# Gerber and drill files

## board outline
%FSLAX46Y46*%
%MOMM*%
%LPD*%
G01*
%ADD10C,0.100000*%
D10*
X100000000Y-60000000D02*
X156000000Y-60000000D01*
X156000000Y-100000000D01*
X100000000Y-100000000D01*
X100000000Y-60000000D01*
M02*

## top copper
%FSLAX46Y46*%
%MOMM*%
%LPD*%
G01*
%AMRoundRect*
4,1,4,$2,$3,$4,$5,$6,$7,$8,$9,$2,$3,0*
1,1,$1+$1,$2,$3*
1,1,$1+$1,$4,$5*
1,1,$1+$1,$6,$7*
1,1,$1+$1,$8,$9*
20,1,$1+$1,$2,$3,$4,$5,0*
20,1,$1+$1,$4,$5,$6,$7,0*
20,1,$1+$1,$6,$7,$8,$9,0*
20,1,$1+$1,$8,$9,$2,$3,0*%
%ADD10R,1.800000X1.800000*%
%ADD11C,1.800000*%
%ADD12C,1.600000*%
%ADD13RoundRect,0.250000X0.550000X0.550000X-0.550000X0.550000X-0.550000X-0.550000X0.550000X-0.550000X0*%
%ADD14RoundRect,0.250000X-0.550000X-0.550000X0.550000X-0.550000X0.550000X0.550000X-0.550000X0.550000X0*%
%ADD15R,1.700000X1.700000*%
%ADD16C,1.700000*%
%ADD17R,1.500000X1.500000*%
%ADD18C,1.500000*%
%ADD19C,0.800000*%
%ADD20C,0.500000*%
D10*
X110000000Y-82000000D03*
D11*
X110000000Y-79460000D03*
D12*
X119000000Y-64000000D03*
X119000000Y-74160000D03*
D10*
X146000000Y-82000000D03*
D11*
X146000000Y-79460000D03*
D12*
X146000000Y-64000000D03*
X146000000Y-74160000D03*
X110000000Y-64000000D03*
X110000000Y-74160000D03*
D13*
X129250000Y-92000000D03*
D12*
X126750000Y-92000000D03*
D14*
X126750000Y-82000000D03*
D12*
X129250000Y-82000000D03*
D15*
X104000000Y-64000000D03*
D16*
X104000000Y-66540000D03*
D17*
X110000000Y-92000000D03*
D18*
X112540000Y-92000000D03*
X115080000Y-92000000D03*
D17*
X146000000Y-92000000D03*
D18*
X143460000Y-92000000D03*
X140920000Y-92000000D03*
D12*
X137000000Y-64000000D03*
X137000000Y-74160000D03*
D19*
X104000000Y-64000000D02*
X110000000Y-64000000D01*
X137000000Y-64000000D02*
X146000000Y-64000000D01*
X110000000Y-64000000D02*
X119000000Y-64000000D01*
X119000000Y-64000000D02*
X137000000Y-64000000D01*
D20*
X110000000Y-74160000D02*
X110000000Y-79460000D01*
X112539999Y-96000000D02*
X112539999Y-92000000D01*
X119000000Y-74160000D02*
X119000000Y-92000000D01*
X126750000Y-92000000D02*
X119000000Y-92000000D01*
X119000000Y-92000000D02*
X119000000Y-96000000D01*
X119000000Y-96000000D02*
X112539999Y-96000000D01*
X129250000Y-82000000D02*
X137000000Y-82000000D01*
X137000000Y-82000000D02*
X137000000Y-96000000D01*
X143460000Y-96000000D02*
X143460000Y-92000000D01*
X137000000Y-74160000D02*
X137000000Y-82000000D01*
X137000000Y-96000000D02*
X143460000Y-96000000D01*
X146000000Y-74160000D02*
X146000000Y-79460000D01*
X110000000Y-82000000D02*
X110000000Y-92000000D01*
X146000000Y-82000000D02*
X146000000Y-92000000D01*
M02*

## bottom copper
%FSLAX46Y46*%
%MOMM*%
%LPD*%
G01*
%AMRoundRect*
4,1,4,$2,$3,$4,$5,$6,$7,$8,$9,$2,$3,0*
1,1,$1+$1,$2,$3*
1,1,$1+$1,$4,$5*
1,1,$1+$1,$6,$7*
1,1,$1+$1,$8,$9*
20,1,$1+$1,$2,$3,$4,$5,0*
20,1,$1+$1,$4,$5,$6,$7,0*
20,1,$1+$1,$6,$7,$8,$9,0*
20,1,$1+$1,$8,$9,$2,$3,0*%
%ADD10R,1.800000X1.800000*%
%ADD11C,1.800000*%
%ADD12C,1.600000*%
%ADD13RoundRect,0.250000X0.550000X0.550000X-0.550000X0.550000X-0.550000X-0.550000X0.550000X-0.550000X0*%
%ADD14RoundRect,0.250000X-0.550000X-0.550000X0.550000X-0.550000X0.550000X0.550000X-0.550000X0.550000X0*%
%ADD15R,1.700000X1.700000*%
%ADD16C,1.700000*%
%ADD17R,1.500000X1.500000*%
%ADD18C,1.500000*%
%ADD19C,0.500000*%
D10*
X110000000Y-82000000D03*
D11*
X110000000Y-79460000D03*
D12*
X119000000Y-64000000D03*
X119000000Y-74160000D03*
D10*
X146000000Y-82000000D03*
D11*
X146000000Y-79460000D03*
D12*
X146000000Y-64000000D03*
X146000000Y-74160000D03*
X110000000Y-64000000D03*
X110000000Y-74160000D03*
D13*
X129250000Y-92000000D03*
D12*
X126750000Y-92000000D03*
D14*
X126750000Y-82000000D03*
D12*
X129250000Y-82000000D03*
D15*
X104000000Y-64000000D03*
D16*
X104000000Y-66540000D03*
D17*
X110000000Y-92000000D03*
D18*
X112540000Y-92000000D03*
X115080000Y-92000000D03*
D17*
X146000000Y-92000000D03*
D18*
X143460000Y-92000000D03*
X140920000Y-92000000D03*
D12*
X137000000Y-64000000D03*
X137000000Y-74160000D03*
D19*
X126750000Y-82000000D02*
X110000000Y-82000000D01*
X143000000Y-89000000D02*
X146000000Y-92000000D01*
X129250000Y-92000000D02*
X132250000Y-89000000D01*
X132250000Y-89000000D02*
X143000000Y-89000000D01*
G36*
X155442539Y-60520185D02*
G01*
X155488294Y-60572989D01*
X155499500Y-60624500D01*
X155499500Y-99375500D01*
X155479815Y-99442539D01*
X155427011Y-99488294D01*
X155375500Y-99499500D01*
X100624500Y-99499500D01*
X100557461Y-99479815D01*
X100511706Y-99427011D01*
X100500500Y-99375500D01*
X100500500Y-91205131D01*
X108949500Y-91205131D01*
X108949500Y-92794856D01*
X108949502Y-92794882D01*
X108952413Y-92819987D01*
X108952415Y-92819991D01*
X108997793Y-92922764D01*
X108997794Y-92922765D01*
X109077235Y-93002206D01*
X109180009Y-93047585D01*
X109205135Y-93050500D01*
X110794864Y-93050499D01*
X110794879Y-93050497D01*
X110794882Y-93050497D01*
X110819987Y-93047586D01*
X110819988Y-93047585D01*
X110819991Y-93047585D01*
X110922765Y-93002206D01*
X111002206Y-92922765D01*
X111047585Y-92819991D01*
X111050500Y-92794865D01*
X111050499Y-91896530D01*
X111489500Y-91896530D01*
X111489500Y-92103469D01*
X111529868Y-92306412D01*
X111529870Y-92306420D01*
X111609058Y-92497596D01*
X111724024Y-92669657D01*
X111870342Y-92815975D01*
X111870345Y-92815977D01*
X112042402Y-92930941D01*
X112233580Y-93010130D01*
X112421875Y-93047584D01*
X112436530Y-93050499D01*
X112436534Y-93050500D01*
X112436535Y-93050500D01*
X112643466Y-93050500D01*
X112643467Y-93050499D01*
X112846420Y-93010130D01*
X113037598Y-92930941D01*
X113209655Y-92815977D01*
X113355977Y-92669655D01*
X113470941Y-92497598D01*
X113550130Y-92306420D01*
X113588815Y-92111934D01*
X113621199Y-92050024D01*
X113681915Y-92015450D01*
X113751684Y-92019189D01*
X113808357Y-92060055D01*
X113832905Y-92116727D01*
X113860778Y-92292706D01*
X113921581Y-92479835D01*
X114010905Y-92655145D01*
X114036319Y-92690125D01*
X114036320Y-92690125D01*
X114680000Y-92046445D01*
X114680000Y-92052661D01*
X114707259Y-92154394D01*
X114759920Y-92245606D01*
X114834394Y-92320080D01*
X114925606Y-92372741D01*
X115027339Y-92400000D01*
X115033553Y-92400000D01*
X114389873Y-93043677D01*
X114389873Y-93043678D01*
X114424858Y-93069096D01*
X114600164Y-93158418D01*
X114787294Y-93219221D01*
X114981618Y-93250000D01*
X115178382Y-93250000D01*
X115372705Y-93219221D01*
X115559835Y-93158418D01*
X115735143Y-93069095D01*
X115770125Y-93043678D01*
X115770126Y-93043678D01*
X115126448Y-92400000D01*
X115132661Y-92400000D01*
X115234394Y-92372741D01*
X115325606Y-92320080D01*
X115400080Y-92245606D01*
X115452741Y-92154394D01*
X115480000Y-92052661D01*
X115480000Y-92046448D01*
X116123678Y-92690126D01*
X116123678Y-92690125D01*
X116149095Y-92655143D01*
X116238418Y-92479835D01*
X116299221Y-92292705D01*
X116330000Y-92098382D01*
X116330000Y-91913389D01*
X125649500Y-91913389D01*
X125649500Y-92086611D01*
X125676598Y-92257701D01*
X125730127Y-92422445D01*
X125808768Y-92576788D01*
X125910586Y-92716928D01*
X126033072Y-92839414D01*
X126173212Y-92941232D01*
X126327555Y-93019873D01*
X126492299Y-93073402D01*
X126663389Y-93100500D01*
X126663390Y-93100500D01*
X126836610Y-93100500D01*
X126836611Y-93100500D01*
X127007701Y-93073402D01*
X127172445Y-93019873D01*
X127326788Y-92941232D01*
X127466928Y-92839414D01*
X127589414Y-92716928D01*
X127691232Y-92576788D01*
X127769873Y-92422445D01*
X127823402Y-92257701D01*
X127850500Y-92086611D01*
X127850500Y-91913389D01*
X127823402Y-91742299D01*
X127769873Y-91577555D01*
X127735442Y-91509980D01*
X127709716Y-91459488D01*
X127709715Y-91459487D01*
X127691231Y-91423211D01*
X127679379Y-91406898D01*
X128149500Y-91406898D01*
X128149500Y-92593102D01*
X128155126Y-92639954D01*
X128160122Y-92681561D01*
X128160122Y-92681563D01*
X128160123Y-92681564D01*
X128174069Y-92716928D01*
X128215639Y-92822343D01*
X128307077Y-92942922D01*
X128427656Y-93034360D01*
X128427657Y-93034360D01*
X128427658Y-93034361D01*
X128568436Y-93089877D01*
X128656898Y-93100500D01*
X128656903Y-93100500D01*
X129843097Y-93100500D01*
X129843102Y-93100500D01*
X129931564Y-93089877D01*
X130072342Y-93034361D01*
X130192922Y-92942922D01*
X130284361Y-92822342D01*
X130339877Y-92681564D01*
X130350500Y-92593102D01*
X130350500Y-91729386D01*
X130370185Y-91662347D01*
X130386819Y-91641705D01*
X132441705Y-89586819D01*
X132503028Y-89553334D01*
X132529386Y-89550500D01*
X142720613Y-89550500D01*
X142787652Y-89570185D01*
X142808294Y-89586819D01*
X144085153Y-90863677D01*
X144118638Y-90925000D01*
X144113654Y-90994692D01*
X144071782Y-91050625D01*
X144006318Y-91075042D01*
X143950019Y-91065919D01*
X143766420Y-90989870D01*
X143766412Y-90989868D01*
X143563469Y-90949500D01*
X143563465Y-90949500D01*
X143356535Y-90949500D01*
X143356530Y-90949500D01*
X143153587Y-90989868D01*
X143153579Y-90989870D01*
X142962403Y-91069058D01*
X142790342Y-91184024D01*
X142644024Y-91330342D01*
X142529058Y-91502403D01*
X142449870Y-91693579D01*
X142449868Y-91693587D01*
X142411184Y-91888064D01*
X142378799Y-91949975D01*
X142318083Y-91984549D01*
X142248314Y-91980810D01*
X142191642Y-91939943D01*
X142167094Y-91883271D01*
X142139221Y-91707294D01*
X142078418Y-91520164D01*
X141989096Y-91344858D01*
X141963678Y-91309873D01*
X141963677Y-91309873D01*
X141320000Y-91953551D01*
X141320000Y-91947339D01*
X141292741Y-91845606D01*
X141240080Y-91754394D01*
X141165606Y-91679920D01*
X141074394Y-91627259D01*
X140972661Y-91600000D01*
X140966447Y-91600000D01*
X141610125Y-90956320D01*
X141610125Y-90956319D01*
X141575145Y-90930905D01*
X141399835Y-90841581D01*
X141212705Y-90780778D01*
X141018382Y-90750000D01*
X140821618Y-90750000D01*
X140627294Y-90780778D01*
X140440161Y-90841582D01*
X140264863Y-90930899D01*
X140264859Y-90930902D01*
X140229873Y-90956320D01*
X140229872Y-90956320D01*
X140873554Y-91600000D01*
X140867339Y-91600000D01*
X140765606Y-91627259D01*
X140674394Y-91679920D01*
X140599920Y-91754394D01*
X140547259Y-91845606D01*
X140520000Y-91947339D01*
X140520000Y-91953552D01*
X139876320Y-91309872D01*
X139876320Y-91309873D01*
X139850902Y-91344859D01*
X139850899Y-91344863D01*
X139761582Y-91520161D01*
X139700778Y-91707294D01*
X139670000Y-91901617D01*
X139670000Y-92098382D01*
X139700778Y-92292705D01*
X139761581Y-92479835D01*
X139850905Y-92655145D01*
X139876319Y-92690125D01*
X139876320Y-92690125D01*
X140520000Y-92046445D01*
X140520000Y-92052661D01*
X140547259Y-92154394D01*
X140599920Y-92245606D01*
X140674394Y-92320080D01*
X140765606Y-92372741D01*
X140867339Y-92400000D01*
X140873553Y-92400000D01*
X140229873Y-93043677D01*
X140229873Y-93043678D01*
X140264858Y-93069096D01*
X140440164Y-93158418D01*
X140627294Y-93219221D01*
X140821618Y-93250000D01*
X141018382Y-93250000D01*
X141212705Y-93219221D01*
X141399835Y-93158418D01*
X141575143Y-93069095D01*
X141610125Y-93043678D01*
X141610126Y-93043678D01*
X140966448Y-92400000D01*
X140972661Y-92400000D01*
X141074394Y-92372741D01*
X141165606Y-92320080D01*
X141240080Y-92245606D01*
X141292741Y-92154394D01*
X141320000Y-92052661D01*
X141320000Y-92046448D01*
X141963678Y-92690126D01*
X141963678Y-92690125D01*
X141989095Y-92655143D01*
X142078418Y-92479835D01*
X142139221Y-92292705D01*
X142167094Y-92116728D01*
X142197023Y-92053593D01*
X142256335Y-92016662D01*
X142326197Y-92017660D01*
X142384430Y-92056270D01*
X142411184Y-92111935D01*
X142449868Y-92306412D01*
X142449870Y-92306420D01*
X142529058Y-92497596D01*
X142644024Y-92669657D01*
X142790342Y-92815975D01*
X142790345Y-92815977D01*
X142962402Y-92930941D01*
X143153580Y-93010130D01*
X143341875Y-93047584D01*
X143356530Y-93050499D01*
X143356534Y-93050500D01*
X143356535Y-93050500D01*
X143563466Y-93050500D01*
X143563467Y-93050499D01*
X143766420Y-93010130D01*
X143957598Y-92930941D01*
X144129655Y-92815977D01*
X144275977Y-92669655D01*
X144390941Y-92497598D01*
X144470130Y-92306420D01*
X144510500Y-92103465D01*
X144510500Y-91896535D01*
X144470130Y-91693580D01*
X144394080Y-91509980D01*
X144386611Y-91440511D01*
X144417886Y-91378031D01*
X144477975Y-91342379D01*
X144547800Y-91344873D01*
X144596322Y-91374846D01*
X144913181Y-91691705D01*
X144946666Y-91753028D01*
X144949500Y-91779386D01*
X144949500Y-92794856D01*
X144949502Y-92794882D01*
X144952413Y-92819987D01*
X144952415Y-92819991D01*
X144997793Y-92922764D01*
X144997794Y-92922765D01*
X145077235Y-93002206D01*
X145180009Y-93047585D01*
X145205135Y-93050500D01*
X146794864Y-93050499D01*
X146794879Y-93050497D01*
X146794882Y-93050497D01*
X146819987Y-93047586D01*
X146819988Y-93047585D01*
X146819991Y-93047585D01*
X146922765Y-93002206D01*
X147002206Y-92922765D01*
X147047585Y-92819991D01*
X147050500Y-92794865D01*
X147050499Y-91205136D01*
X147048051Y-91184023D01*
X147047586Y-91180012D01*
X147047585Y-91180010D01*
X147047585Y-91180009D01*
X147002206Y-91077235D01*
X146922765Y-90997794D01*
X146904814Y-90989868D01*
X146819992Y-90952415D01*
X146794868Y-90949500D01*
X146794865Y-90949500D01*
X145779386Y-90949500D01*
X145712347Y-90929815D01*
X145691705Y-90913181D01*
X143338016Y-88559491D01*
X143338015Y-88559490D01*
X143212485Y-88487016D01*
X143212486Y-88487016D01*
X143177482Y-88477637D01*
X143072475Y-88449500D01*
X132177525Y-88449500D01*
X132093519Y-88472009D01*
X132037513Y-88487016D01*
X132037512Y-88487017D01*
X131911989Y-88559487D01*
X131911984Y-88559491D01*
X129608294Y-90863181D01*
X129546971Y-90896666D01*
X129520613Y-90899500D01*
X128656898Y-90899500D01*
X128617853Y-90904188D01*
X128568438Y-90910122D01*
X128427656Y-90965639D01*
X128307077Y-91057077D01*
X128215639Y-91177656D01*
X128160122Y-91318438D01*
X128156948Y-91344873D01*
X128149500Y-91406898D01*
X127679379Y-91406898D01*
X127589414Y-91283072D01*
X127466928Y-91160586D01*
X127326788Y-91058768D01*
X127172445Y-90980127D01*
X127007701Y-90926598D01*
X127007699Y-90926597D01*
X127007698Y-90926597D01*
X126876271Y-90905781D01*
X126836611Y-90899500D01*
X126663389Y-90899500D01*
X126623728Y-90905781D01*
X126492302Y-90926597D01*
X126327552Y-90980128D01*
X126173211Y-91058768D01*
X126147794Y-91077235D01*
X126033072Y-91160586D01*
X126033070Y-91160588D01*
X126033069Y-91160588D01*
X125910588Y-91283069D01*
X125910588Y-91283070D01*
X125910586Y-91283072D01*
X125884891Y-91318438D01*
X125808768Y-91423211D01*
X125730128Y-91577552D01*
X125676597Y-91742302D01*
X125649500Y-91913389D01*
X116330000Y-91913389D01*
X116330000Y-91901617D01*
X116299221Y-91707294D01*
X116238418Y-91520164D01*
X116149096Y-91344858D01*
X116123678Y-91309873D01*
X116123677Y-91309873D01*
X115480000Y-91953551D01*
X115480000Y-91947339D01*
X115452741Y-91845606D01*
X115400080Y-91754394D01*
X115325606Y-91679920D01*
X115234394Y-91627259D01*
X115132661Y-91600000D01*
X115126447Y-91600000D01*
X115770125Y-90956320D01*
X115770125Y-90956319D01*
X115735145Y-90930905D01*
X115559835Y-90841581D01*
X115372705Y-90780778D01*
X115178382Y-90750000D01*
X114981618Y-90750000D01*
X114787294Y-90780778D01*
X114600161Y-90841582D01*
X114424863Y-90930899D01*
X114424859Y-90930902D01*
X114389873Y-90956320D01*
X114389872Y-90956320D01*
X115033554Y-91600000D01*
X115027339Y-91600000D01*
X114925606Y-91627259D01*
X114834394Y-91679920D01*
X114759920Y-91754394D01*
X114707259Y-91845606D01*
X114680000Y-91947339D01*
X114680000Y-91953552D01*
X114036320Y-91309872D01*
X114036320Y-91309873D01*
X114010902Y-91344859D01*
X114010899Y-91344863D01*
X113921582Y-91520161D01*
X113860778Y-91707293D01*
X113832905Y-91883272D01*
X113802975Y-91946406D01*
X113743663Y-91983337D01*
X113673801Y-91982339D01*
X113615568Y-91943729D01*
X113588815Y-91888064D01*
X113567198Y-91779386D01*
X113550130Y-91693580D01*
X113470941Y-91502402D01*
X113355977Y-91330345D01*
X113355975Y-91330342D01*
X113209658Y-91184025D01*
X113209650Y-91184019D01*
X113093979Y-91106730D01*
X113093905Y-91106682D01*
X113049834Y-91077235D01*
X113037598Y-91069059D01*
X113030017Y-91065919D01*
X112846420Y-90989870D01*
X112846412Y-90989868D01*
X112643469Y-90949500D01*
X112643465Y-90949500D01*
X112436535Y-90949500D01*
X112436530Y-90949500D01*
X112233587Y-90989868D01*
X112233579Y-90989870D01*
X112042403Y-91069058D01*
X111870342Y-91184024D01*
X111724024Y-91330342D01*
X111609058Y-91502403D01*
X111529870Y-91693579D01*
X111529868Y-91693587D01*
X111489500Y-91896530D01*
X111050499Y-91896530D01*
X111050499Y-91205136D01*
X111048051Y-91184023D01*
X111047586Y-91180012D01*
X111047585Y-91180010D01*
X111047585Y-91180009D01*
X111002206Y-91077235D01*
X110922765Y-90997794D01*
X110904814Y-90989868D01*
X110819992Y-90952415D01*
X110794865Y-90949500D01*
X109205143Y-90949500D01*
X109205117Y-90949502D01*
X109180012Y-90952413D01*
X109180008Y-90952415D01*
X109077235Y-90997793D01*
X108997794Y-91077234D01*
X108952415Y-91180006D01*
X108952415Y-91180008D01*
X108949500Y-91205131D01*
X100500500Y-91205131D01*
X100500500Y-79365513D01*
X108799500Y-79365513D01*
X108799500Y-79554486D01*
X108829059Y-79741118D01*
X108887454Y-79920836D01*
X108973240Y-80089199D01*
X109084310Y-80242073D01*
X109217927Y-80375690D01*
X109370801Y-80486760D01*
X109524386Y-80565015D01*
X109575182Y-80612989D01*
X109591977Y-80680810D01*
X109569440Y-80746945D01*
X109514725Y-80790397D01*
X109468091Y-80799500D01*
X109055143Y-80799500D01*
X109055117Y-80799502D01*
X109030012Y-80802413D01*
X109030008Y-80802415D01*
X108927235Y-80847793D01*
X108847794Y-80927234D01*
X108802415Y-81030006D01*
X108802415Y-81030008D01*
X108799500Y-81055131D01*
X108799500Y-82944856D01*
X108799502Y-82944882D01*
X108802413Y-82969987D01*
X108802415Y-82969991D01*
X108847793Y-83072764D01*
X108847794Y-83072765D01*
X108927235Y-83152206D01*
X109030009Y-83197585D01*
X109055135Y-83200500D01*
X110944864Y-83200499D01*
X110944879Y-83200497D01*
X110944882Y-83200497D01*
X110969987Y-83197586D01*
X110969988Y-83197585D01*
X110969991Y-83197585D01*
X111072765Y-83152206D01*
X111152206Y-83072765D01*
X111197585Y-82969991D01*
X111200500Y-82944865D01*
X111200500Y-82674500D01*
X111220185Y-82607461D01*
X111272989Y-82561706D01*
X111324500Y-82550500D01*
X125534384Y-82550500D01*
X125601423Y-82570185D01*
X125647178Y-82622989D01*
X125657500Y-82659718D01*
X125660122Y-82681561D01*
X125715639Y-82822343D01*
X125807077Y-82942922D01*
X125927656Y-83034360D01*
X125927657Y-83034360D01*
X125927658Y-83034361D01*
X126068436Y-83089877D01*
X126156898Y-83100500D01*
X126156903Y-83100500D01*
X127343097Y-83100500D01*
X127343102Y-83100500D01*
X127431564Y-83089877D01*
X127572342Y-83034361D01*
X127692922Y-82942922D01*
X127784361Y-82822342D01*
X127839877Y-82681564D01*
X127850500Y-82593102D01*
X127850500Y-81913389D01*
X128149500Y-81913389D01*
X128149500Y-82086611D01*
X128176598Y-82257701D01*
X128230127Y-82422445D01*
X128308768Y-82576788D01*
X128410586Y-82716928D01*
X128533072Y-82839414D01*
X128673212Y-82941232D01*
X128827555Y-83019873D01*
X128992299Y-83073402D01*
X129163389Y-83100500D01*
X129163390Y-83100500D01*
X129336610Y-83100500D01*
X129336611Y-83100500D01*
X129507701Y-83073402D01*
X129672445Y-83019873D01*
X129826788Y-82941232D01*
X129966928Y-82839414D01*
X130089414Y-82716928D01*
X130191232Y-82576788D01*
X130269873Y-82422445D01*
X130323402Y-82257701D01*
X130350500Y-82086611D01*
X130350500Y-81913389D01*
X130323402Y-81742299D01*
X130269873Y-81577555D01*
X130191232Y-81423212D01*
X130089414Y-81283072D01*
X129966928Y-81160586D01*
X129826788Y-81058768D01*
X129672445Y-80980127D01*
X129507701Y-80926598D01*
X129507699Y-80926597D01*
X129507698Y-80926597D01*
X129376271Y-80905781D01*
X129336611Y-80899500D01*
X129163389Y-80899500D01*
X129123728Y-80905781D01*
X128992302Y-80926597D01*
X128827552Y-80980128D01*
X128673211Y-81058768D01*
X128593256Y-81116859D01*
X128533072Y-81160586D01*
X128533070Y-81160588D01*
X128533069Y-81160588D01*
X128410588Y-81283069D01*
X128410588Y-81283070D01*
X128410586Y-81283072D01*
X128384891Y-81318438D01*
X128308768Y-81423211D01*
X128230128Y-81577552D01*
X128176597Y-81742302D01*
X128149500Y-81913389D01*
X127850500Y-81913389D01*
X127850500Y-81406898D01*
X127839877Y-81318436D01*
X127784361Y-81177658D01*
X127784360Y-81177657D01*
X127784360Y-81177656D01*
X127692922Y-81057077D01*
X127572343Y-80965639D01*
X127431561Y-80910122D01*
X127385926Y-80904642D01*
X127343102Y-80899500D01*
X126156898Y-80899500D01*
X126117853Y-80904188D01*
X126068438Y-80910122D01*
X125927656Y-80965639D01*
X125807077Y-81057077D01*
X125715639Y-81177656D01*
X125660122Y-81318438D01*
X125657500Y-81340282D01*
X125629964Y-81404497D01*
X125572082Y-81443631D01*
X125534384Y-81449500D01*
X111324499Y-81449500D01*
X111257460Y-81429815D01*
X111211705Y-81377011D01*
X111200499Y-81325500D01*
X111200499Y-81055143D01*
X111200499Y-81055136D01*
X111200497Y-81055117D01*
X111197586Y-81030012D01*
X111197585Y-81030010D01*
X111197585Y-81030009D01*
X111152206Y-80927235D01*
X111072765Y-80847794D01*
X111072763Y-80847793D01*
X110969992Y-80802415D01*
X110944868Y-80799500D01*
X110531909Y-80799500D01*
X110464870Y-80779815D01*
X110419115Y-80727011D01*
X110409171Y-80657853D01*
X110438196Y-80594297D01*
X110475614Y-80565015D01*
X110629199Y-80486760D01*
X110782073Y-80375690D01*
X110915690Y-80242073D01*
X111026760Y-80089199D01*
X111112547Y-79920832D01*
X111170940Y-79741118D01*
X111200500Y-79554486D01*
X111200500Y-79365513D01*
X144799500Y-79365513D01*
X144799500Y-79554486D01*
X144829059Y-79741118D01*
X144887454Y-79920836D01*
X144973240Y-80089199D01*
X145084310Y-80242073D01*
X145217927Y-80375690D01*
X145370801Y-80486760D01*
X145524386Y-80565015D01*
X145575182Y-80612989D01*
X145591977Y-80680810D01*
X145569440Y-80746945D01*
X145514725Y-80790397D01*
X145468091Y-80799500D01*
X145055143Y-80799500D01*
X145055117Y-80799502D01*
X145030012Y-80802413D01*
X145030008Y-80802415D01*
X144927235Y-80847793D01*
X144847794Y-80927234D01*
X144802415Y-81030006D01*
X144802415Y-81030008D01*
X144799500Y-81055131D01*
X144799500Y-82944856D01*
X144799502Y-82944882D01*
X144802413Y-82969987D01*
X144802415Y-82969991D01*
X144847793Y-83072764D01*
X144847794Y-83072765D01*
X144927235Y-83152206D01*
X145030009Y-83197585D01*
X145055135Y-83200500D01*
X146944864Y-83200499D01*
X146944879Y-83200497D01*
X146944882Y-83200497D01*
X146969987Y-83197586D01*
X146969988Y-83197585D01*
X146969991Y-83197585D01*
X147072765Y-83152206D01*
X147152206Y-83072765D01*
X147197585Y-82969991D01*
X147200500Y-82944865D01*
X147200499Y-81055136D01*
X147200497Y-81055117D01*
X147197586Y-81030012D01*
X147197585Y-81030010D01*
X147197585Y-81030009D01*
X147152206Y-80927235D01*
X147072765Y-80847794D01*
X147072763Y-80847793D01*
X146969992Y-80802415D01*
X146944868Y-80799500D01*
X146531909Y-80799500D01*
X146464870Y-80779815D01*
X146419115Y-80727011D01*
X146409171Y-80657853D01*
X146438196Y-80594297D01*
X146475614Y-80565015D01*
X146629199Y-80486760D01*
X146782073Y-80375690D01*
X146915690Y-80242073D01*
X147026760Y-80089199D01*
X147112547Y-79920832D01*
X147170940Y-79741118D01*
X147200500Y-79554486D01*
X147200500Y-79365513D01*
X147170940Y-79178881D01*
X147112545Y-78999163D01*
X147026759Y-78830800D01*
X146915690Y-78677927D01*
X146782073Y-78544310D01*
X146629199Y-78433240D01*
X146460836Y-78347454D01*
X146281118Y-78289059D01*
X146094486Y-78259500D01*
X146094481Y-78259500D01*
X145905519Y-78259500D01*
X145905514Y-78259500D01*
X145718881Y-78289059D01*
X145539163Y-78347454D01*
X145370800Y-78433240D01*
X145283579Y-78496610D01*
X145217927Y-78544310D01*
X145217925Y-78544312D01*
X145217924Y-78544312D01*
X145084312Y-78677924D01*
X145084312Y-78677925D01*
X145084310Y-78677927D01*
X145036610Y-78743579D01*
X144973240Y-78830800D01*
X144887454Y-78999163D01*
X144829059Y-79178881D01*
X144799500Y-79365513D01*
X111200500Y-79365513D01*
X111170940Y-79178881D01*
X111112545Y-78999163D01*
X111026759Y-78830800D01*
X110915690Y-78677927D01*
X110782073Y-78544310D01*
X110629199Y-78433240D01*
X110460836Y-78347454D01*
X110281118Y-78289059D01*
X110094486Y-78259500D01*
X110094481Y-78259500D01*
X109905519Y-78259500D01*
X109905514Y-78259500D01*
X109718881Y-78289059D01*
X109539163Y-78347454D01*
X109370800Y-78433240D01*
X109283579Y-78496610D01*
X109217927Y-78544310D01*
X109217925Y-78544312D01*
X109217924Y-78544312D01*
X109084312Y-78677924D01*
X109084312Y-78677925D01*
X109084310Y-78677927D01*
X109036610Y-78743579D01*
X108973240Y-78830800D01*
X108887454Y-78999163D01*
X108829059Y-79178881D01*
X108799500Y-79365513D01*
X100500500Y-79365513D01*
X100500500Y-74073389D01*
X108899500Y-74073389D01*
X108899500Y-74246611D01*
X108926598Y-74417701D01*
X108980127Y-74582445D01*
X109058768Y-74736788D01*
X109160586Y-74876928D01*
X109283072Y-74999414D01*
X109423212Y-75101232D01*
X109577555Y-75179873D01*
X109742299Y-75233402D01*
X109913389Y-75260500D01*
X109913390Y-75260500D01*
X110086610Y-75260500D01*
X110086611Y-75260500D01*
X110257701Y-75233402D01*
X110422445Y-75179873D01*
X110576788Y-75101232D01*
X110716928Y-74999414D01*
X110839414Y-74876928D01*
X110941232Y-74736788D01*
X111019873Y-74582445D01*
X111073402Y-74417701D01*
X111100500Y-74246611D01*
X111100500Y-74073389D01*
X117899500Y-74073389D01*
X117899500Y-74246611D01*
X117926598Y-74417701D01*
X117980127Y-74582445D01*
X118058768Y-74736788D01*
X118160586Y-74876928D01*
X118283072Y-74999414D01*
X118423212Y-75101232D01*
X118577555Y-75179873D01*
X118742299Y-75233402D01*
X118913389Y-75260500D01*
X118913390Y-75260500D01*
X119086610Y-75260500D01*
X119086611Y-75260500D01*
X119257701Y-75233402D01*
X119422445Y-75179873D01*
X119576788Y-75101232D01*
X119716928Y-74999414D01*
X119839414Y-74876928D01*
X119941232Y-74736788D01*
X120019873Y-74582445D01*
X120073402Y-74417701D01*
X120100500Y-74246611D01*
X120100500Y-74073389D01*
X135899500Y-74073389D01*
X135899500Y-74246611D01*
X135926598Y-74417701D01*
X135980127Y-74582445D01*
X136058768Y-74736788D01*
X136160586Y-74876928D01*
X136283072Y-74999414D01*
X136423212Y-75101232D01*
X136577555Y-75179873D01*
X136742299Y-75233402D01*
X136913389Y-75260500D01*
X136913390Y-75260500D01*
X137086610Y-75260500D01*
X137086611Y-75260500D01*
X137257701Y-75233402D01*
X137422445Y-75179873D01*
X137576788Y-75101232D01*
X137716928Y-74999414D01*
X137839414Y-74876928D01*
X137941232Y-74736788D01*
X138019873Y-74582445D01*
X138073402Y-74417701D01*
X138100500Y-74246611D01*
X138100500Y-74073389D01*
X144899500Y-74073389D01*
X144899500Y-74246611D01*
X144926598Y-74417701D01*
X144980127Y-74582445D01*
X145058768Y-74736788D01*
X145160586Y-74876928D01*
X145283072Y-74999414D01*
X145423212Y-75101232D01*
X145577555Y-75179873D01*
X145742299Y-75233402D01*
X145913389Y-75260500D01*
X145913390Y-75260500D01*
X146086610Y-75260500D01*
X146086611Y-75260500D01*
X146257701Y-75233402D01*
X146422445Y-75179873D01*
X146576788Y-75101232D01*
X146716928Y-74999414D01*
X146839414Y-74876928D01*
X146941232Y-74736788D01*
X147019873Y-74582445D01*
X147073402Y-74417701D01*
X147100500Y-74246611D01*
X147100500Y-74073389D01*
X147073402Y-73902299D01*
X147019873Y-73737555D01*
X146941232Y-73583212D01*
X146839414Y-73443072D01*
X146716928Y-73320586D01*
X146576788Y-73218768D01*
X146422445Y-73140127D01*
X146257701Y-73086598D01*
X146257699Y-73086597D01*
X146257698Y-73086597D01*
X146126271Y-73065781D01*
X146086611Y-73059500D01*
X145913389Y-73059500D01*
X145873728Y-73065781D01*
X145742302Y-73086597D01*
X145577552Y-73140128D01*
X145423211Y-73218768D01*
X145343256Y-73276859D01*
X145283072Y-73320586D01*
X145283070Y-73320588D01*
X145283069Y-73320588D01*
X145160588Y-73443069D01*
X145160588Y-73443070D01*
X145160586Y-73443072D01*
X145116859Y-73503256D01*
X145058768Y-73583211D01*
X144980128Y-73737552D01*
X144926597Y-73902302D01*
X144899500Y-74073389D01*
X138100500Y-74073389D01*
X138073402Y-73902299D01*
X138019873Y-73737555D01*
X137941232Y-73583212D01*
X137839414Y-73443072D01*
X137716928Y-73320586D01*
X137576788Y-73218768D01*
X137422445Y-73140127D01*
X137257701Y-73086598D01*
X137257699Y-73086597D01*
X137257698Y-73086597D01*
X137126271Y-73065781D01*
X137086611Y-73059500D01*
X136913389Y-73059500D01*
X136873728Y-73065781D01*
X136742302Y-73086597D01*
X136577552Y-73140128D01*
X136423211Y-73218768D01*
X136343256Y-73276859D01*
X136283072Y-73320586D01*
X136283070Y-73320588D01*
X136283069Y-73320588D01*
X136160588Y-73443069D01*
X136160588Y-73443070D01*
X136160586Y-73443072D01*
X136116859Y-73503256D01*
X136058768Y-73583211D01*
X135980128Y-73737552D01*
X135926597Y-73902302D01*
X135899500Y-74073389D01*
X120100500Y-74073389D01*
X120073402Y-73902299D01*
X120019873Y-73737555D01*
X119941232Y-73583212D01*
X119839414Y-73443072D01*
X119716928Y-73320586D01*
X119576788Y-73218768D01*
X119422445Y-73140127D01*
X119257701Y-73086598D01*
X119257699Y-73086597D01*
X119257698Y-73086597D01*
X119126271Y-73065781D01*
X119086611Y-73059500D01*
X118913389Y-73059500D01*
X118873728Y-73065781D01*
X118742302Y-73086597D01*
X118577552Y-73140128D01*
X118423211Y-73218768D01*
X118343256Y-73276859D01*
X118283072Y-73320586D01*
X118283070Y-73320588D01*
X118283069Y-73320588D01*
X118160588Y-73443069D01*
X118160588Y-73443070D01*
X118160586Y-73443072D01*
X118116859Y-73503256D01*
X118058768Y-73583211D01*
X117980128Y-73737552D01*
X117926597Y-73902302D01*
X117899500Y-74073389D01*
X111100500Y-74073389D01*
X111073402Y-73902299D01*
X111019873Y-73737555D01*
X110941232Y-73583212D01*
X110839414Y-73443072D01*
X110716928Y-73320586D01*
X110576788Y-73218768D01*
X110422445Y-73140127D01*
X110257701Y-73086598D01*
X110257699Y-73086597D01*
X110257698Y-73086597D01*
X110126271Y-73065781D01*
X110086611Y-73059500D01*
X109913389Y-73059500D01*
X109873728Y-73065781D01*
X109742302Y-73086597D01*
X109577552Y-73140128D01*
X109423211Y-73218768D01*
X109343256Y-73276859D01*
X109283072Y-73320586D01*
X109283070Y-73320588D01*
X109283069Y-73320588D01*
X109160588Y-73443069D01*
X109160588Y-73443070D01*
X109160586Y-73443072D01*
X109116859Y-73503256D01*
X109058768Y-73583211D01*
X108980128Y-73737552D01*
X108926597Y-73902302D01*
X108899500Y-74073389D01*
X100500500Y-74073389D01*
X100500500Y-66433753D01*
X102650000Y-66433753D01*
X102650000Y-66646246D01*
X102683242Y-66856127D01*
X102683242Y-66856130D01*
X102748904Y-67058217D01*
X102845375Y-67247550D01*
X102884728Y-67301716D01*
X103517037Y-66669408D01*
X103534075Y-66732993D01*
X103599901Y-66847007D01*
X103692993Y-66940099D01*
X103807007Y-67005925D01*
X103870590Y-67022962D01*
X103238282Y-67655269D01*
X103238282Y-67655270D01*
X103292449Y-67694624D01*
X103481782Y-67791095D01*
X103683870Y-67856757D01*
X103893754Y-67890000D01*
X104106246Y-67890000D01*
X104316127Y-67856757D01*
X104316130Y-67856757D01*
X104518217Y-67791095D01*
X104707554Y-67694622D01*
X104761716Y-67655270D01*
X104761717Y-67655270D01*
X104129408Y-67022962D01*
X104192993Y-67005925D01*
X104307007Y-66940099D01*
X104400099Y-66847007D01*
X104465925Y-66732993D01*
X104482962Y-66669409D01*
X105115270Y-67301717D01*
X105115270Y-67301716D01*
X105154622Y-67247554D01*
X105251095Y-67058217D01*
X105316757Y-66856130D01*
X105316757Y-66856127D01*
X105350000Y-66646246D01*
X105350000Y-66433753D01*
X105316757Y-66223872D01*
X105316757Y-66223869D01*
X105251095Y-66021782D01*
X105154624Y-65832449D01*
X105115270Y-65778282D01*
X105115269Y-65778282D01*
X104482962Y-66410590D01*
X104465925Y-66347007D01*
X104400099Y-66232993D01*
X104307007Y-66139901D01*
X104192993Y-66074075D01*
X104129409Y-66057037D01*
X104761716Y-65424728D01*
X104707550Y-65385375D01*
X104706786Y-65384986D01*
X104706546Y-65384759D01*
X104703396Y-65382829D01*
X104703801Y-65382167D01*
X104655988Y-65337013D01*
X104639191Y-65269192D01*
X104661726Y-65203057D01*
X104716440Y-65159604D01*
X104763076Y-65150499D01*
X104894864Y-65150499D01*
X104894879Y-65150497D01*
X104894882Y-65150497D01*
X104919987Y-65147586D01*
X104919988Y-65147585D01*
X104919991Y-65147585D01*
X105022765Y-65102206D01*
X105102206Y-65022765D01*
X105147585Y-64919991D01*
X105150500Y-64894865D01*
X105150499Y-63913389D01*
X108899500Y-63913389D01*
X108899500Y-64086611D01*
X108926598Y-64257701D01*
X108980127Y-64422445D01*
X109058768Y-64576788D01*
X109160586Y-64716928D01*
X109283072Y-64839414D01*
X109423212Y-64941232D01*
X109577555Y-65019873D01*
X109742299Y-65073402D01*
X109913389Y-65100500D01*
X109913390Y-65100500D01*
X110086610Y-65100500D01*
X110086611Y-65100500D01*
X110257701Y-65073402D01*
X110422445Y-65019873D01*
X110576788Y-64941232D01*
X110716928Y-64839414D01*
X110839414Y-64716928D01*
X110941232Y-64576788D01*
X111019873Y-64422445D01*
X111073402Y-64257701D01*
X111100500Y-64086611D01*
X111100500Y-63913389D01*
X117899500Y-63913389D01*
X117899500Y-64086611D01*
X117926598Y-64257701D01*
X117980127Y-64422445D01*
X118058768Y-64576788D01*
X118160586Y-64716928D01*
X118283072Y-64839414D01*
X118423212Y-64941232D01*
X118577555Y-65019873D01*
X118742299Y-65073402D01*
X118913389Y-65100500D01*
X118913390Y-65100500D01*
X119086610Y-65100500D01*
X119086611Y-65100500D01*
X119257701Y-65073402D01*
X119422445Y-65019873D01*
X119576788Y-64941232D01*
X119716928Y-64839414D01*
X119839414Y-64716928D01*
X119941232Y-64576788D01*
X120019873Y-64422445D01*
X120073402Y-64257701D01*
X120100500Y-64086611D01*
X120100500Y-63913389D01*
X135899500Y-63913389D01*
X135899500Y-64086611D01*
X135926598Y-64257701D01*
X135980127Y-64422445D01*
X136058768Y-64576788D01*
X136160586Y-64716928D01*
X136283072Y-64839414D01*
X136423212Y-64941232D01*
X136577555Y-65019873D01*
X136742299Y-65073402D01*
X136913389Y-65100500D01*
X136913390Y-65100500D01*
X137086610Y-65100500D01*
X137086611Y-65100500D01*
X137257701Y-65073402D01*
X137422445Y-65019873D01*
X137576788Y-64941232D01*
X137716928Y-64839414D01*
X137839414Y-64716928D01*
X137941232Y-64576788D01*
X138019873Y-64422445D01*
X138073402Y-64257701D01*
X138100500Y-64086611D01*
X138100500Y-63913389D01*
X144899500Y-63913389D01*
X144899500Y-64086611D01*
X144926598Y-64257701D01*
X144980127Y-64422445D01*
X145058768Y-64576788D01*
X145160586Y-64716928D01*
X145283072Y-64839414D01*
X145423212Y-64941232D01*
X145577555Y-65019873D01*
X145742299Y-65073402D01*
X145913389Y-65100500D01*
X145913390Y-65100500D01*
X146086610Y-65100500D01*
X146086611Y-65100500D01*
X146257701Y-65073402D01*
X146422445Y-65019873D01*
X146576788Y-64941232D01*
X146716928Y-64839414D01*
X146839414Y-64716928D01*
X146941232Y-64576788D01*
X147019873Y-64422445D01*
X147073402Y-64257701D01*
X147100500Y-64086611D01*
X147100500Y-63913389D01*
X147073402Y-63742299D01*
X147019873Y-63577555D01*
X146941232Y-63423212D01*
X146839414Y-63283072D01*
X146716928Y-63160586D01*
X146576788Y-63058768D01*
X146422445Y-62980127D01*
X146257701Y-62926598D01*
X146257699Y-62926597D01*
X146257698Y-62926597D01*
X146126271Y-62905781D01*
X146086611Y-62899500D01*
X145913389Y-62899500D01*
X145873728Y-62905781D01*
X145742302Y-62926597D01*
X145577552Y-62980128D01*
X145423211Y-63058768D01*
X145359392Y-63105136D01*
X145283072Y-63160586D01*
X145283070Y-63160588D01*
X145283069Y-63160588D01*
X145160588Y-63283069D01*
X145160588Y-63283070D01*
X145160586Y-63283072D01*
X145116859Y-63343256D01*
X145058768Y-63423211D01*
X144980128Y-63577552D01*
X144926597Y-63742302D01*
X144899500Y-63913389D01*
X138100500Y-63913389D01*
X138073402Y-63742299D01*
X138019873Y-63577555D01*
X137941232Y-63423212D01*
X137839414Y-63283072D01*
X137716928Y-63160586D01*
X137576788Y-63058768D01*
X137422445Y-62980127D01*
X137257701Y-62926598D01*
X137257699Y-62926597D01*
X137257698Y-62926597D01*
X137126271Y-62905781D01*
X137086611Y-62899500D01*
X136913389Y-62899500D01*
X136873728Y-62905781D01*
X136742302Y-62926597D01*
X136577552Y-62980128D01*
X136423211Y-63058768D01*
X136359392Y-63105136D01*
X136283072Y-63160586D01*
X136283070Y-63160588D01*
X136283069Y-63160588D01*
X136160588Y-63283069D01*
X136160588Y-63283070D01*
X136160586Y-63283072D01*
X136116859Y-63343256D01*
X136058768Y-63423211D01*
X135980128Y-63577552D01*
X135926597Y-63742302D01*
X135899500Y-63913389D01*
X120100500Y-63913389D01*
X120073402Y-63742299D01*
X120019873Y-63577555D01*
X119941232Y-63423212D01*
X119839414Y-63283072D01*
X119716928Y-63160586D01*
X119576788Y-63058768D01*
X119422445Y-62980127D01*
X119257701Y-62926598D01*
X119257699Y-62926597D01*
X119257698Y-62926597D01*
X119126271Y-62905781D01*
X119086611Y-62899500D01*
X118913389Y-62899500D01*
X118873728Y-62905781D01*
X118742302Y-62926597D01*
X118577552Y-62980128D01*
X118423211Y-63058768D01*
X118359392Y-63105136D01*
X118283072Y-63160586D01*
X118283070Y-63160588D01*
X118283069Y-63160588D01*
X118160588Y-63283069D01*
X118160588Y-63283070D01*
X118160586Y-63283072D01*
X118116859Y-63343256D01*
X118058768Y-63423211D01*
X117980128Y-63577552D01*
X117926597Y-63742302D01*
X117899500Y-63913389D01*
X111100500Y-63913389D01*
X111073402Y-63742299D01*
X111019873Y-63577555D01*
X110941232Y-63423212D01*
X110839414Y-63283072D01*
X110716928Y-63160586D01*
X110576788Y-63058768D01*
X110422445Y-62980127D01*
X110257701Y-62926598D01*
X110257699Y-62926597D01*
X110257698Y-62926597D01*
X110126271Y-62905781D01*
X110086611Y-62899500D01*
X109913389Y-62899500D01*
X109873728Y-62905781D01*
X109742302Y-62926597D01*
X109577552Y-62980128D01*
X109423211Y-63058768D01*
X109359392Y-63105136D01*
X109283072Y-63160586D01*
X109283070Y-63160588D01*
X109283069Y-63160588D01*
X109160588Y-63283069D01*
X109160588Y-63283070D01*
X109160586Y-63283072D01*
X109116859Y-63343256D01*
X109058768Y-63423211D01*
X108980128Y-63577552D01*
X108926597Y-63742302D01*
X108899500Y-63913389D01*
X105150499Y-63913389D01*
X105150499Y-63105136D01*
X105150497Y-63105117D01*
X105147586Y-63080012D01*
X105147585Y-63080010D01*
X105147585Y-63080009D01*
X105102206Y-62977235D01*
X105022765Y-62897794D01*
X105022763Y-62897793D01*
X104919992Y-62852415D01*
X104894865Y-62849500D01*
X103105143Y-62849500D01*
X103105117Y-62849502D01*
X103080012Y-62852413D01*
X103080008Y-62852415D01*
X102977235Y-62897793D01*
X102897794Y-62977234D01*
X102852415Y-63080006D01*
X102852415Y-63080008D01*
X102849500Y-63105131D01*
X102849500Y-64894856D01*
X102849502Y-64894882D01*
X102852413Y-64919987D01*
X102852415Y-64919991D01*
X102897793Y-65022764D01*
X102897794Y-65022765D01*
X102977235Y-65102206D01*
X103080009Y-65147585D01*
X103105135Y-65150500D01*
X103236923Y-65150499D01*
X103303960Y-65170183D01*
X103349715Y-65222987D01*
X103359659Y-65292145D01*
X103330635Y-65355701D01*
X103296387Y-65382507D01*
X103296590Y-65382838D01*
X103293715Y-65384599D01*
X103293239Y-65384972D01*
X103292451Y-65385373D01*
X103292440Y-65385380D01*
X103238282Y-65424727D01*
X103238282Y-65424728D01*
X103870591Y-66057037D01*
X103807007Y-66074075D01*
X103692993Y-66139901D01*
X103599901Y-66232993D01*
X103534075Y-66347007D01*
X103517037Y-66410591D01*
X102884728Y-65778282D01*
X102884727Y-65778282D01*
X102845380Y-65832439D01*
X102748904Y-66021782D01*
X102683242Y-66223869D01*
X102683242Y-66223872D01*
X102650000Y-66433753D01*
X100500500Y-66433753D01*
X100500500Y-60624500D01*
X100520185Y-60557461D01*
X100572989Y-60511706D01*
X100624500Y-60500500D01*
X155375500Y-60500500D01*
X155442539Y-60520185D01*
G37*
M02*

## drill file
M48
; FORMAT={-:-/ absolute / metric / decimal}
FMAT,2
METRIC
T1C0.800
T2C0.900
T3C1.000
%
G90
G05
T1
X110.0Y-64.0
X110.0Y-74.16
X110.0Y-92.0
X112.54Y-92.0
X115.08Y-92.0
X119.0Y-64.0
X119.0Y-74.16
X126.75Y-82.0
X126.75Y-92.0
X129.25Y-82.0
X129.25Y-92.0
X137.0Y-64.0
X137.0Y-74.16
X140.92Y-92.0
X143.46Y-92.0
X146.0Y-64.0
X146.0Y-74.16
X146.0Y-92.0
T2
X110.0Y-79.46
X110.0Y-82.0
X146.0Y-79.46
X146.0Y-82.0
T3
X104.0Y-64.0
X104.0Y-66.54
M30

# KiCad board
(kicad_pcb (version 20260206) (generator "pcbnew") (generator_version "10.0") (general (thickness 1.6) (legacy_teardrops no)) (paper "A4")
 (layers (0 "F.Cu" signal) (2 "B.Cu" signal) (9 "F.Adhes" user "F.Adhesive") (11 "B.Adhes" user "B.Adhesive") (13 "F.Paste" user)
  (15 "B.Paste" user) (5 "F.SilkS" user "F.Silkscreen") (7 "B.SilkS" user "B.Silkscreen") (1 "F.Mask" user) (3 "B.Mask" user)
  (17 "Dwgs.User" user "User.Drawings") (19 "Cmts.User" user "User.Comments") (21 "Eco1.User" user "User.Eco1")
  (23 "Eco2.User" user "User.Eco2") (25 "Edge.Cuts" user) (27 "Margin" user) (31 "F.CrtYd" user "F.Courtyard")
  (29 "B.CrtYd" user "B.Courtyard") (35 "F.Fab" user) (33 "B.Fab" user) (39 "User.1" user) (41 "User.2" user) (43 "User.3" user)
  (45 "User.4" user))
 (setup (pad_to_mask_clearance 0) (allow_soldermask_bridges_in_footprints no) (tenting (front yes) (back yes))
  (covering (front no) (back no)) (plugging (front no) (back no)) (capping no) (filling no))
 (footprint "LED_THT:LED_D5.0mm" (layer "F.Cu") (at 110 82 90)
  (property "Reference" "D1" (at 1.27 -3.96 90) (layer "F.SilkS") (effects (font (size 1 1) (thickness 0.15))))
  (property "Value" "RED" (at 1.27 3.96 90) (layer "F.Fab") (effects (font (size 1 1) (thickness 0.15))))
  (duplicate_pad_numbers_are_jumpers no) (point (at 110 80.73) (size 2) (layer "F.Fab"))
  (pad "1" thru_hole rect (at 0 0 90) (size 1.8 1.8) (drill 0.9) (layers "*.Cu" "*.Mask") (remove_unused_layers no) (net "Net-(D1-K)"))
  (pad "2" thru_hole circle (at 2.54 0 90) (size 1.8 1.8) (drill 0.9) (layers "*.Cu" "*.Mask") (remove_unused_layers no) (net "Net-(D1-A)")))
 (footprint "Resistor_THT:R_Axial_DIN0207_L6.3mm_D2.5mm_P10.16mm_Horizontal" (layer "F.Cu") (at 119 64 -90)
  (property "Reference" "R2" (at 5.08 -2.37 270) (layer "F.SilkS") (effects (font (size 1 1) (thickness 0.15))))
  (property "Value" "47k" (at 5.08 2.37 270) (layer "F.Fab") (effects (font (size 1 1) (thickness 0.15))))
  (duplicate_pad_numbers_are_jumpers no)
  (pad "1" thru_hole circle (at 0 0 270) (size 1.6 1.6) (drill 0.8) (layers "*.Cu" "*.Mask") (remove_unused_layers no) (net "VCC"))
  (pad "2" thru_hole circle (at 10.16 0 270) (size 1.6 1.6) (drill 0.8) (layers "*.Cu" "*.Mask") (remove_unused_layers no)
   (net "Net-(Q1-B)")))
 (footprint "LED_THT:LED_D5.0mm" (layer "F.Cu") (at 146 82 90)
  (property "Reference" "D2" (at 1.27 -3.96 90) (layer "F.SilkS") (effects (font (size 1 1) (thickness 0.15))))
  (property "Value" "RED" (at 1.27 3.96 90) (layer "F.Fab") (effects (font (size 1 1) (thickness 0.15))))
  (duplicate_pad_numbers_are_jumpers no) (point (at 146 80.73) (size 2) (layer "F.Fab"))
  (pad "1" thru_hole rect (at 0 0 90) (size 1.8 1.8) (drill 0.9) (layers "*.Cu" "*.Mask") (remove_unused_layers no) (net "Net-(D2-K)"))
  (pad "2" thru_hole circle (at 2.54 0 90) (size 1.8 1.8) (drill 0.9) (layers "*.Cu" "*.Mask") (remove_unused_layers no) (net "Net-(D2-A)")))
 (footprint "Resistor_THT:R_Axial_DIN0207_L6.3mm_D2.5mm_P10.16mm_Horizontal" (layer "F.Cu") (at 146 64 -90)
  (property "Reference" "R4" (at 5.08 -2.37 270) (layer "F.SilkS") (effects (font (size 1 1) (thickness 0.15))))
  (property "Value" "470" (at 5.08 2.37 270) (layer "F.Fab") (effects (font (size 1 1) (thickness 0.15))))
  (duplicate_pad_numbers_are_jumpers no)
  (pad "1" thru_hole circle (at 0 0 270) (size 1.6 1.6) (drill 0.8) (layers "*.Cu" "*.Mask") (remove_unused_layers no) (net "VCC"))
  (pad "2" thru_hole circle (at 10.16 0 270) (size 1.6 1.6) (drill 0.8) (layers "*.Cu" "*.Mask") (remove_unused_layers no)
   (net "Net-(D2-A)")))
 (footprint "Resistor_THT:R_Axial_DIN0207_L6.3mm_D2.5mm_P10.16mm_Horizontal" (layer "F.Cu") (at 110 64 -90)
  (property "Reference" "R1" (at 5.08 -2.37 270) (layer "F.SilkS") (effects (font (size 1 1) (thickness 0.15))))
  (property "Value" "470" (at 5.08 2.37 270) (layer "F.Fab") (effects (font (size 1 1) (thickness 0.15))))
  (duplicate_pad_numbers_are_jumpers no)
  (pad "1" thru_hole circle (at 0 0 270) (size 1.6 1.6) (drill 0.8) (layers "*.Cu" "*.Mask") (remove_unused_layers no) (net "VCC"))
  (pad "2" thru_hole circle (at 10.16 0 270) (size 1.6 1.6) (drill 0.8) (layers "*.Cu" "*.Mask") (remove_unused_layers no)
   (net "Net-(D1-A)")))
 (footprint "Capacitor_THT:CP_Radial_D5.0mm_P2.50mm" (layer "F.Cu") (at 129.25 92 180)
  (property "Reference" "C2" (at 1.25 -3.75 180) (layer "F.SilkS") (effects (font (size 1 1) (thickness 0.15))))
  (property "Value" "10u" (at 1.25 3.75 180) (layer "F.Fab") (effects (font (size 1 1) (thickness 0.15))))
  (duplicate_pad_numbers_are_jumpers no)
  (pad "1" thru_hole roundrect (at 0 0 180) (size 1.6 1.6) (drill 0.8) (layers "*.Cu" "*.Mask") (remove_unused_layers no)
   (roundrect_rratio 0.15625) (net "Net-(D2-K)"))
  (pad "2" thru_hole circle (at 2.5 0 180) (size 1.6 1.6) (drill 0.8) (layers "*.Cu" "*.Mask") (remove_unused_layers no) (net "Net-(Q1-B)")))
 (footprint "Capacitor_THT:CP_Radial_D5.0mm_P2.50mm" (layer "F.Cu") (at 126.75 82)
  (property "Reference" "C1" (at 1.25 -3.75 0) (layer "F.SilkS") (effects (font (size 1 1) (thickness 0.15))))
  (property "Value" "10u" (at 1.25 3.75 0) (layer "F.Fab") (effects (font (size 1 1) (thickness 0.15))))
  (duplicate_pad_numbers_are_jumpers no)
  (pad "1" thru_hole roundrect (at 0 0) (size 1.6 1.6) (drill 0.8) (layers "*.Cu" "*.Mask") (remove_unused_layers no)
   (roundrect_rratio 0.15625) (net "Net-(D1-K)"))
  (pad "2" thru_hole circle (at 2.5 0) (size 1.6 1.6) (drill 0.8) (layers "*.Cu" "*.Mask") (remove_unused_layers no) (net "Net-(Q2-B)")))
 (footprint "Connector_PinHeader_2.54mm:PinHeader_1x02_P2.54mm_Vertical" (layer "F.Cu") (at 104 64)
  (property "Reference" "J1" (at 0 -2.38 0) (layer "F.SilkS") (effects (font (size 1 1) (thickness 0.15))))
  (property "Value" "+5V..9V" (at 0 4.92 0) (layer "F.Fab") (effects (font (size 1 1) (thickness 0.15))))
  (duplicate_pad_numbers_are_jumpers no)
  (pad "1" thru_hole rect (at 0 0) (size 1.7 1.7) (drill 1) (layers "*.Cu" "*.Mask") (remove_unused_layers no) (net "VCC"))
  (pad "2" thru_hole circle (at 0 2.54) (size 1.7 1.7) (drill 1) (layers "*.Cu" "*.Mask") (remove_unused_layers no) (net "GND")))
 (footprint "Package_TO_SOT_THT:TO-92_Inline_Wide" (layer "F.Cu") (at 110 92)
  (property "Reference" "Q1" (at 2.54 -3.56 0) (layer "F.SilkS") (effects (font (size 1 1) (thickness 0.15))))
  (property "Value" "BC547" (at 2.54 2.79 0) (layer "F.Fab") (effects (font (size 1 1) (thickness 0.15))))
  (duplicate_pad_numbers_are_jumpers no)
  (pad "1" thru_hole rect (at 0 0) (size 1.5 1.5) (drill 0.8) (layers "*.Cu" "*.Mask") (remove_unused_layers no) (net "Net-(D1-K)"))
  (pad "2" thru_hole circle (at 2.54 0) (size 1.5 1.5) (drill 0.8) (layers "*.Cu" "*.Mask") (remove_unused_layers no) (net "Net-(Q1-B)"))
  (pad "3" thru_hole circle (at 5.08 0) (size 1.5 1.5) (drill 0.8) (layers "*.Cu" "*.Mask") (remove_unused_layers no) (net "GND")))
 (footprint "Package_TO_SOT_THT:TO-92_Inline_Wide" (layer "F.Cu") (at 146 92 180)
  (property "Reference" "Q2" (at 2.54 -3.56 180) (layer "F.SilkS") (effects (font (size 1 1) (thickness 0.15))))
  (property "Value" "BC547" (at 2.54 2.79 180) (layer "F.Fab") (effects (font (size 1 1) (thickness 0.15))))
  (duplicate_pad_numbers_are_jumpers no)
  (pad "1" thru_hole rect (at 0 0 180) (size 1.5 1.5) (drill 0.8) (layers "*.Cu" "*.Mask") (remove_unused_layers no) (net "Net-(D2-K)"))
  (pad "2" thru_hole circle (at 2.54 0 180) (size 1.5 1.5) (drill 0.8) (layers "*.Cu" "*.Mask") (remove_unused_layers no) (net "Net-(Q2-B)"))
  (pad "3" thru_hole circle (at 5.08 0 180) (size 1.5 1.5) (drill 0.8) (layers "*.Cu" "*.Mask") (remove_unused_layers no) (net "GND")))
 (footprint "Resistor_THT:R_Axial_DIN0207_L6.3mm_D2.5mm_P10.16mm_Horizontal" (layer "F.Cu") (at 137 64 -90)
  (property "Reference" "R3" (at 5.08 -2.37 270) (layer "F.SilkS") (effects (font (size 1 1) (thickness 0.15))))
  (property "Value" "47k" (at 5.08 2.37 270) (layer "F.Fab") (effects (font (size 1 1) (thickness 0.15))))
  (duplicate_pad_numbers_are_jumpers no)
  (pad "1" thru_hole circle (at 0 0 270) (size 1.6 1.6) (drill 0.8) (layers "*.Cu" "*.Mask") (remove_unused_layers no) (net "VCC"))
  (pad "2" thru_hole circle (at 10.16 0 270) (size 1.6 1.6) (drill 0.8) (layers "*.Cu" "*.Mask") (remove_unused_layers no)
   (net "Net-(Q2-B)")))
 (gr_rect (start 100 60) (end 156 100) (stroke (width 0.1) (type default)) (fill no) (layer "Edge.Cuts"))
 (segment (start 104 64) (end 110 64) (width 0.8) (layer "F.Cu") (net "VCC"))
 (segment (start 137 64) (end 146 64) (width 0.8) (layer "F.Cu") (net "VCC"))
 (segment (start 110 64) (end 119 64) (width 0.8) (layer "F.Cu") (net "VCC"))
 (segment (start 119 64) (end 137 64) (width 0.8) (layer "F.Cu") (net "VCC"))
 (segment (start 110 74.16) (end 110 79.46) (width 0.5) (layer "F.Cu") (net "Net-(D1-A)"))
 (segment (start 112.539999 96) (end 112.539999 92) (width 0.5) (layer "F.Cu") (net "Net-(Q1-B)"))
 (segment (start 119 74.16) (end 119 92) (width 0.5) (layer "F.Cu") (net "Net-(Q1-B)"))
 (segment (start 126.75 92) (end 119 92) (width 0.5) (layer "F.Cu") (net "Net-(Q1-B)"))
 (segment (start 119 92) (end 119 96) (width 0.5) (layer "F.Cu") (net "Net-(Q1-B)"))
 (segment (start 119 96) (end 112.539999 96) (width 0.5) (layer "F.Cu") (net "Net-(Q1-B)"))
 (segment (start 129.25 82) (end 137 82) (width 0.5) (layer "F.Cu") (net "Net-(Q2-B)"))
 (segment (start 137 82) (end 137 96) (width 0.5) (layer "F.Cu") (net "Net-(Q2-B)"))
 (segment (start 143.46 96) (end 143.46 92) (width 0.5) (layer "F.Cu") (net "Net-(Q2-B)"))
 (segment (start 137 74.16) (end 137 82) (width 0.5) (layer "F.Cu") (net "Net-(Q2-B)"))
 (segment (start 137 96) (end 143.46 96) (width 0.5) (layer "F.Cu") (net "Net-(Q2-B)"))
 (segment (start 146 74.16) (end 146 79.46) (width 0.5) (layer "F.Cu") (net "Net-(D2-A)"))
 (segment (start 110 82) (end 110 92) (width 0.5) (layer "F.Cu") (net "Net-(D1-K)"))
 (segment (start 126.75 82) (end 110 82) (width 0.5) (layer "B.Cu") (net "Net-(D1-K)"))
 (segment (start 146 82) (end 146 92) (width 0.5) (layer "F.Cu") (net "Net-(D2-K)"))
 (segment (start 143 89) (end 146 92) (width 0.5) (layer "B.Cu") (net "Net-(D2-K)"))
 (segment (start 129.25 92) (end 132.25 89) (width 0.5) (layer "B.Cu") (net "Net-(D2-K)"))
 (segment (start 132.25 89) (end 143 89) (width 0.5) (layer "B.Cu") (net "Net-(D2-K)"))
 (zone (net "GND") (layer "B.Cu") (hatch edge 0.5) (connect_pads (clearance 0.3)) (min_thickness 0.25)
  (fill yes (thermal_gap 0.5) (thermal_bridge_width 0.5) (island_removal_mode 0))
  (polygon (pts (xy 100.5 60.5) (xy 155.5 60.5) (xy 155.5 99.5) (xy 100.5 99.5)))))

